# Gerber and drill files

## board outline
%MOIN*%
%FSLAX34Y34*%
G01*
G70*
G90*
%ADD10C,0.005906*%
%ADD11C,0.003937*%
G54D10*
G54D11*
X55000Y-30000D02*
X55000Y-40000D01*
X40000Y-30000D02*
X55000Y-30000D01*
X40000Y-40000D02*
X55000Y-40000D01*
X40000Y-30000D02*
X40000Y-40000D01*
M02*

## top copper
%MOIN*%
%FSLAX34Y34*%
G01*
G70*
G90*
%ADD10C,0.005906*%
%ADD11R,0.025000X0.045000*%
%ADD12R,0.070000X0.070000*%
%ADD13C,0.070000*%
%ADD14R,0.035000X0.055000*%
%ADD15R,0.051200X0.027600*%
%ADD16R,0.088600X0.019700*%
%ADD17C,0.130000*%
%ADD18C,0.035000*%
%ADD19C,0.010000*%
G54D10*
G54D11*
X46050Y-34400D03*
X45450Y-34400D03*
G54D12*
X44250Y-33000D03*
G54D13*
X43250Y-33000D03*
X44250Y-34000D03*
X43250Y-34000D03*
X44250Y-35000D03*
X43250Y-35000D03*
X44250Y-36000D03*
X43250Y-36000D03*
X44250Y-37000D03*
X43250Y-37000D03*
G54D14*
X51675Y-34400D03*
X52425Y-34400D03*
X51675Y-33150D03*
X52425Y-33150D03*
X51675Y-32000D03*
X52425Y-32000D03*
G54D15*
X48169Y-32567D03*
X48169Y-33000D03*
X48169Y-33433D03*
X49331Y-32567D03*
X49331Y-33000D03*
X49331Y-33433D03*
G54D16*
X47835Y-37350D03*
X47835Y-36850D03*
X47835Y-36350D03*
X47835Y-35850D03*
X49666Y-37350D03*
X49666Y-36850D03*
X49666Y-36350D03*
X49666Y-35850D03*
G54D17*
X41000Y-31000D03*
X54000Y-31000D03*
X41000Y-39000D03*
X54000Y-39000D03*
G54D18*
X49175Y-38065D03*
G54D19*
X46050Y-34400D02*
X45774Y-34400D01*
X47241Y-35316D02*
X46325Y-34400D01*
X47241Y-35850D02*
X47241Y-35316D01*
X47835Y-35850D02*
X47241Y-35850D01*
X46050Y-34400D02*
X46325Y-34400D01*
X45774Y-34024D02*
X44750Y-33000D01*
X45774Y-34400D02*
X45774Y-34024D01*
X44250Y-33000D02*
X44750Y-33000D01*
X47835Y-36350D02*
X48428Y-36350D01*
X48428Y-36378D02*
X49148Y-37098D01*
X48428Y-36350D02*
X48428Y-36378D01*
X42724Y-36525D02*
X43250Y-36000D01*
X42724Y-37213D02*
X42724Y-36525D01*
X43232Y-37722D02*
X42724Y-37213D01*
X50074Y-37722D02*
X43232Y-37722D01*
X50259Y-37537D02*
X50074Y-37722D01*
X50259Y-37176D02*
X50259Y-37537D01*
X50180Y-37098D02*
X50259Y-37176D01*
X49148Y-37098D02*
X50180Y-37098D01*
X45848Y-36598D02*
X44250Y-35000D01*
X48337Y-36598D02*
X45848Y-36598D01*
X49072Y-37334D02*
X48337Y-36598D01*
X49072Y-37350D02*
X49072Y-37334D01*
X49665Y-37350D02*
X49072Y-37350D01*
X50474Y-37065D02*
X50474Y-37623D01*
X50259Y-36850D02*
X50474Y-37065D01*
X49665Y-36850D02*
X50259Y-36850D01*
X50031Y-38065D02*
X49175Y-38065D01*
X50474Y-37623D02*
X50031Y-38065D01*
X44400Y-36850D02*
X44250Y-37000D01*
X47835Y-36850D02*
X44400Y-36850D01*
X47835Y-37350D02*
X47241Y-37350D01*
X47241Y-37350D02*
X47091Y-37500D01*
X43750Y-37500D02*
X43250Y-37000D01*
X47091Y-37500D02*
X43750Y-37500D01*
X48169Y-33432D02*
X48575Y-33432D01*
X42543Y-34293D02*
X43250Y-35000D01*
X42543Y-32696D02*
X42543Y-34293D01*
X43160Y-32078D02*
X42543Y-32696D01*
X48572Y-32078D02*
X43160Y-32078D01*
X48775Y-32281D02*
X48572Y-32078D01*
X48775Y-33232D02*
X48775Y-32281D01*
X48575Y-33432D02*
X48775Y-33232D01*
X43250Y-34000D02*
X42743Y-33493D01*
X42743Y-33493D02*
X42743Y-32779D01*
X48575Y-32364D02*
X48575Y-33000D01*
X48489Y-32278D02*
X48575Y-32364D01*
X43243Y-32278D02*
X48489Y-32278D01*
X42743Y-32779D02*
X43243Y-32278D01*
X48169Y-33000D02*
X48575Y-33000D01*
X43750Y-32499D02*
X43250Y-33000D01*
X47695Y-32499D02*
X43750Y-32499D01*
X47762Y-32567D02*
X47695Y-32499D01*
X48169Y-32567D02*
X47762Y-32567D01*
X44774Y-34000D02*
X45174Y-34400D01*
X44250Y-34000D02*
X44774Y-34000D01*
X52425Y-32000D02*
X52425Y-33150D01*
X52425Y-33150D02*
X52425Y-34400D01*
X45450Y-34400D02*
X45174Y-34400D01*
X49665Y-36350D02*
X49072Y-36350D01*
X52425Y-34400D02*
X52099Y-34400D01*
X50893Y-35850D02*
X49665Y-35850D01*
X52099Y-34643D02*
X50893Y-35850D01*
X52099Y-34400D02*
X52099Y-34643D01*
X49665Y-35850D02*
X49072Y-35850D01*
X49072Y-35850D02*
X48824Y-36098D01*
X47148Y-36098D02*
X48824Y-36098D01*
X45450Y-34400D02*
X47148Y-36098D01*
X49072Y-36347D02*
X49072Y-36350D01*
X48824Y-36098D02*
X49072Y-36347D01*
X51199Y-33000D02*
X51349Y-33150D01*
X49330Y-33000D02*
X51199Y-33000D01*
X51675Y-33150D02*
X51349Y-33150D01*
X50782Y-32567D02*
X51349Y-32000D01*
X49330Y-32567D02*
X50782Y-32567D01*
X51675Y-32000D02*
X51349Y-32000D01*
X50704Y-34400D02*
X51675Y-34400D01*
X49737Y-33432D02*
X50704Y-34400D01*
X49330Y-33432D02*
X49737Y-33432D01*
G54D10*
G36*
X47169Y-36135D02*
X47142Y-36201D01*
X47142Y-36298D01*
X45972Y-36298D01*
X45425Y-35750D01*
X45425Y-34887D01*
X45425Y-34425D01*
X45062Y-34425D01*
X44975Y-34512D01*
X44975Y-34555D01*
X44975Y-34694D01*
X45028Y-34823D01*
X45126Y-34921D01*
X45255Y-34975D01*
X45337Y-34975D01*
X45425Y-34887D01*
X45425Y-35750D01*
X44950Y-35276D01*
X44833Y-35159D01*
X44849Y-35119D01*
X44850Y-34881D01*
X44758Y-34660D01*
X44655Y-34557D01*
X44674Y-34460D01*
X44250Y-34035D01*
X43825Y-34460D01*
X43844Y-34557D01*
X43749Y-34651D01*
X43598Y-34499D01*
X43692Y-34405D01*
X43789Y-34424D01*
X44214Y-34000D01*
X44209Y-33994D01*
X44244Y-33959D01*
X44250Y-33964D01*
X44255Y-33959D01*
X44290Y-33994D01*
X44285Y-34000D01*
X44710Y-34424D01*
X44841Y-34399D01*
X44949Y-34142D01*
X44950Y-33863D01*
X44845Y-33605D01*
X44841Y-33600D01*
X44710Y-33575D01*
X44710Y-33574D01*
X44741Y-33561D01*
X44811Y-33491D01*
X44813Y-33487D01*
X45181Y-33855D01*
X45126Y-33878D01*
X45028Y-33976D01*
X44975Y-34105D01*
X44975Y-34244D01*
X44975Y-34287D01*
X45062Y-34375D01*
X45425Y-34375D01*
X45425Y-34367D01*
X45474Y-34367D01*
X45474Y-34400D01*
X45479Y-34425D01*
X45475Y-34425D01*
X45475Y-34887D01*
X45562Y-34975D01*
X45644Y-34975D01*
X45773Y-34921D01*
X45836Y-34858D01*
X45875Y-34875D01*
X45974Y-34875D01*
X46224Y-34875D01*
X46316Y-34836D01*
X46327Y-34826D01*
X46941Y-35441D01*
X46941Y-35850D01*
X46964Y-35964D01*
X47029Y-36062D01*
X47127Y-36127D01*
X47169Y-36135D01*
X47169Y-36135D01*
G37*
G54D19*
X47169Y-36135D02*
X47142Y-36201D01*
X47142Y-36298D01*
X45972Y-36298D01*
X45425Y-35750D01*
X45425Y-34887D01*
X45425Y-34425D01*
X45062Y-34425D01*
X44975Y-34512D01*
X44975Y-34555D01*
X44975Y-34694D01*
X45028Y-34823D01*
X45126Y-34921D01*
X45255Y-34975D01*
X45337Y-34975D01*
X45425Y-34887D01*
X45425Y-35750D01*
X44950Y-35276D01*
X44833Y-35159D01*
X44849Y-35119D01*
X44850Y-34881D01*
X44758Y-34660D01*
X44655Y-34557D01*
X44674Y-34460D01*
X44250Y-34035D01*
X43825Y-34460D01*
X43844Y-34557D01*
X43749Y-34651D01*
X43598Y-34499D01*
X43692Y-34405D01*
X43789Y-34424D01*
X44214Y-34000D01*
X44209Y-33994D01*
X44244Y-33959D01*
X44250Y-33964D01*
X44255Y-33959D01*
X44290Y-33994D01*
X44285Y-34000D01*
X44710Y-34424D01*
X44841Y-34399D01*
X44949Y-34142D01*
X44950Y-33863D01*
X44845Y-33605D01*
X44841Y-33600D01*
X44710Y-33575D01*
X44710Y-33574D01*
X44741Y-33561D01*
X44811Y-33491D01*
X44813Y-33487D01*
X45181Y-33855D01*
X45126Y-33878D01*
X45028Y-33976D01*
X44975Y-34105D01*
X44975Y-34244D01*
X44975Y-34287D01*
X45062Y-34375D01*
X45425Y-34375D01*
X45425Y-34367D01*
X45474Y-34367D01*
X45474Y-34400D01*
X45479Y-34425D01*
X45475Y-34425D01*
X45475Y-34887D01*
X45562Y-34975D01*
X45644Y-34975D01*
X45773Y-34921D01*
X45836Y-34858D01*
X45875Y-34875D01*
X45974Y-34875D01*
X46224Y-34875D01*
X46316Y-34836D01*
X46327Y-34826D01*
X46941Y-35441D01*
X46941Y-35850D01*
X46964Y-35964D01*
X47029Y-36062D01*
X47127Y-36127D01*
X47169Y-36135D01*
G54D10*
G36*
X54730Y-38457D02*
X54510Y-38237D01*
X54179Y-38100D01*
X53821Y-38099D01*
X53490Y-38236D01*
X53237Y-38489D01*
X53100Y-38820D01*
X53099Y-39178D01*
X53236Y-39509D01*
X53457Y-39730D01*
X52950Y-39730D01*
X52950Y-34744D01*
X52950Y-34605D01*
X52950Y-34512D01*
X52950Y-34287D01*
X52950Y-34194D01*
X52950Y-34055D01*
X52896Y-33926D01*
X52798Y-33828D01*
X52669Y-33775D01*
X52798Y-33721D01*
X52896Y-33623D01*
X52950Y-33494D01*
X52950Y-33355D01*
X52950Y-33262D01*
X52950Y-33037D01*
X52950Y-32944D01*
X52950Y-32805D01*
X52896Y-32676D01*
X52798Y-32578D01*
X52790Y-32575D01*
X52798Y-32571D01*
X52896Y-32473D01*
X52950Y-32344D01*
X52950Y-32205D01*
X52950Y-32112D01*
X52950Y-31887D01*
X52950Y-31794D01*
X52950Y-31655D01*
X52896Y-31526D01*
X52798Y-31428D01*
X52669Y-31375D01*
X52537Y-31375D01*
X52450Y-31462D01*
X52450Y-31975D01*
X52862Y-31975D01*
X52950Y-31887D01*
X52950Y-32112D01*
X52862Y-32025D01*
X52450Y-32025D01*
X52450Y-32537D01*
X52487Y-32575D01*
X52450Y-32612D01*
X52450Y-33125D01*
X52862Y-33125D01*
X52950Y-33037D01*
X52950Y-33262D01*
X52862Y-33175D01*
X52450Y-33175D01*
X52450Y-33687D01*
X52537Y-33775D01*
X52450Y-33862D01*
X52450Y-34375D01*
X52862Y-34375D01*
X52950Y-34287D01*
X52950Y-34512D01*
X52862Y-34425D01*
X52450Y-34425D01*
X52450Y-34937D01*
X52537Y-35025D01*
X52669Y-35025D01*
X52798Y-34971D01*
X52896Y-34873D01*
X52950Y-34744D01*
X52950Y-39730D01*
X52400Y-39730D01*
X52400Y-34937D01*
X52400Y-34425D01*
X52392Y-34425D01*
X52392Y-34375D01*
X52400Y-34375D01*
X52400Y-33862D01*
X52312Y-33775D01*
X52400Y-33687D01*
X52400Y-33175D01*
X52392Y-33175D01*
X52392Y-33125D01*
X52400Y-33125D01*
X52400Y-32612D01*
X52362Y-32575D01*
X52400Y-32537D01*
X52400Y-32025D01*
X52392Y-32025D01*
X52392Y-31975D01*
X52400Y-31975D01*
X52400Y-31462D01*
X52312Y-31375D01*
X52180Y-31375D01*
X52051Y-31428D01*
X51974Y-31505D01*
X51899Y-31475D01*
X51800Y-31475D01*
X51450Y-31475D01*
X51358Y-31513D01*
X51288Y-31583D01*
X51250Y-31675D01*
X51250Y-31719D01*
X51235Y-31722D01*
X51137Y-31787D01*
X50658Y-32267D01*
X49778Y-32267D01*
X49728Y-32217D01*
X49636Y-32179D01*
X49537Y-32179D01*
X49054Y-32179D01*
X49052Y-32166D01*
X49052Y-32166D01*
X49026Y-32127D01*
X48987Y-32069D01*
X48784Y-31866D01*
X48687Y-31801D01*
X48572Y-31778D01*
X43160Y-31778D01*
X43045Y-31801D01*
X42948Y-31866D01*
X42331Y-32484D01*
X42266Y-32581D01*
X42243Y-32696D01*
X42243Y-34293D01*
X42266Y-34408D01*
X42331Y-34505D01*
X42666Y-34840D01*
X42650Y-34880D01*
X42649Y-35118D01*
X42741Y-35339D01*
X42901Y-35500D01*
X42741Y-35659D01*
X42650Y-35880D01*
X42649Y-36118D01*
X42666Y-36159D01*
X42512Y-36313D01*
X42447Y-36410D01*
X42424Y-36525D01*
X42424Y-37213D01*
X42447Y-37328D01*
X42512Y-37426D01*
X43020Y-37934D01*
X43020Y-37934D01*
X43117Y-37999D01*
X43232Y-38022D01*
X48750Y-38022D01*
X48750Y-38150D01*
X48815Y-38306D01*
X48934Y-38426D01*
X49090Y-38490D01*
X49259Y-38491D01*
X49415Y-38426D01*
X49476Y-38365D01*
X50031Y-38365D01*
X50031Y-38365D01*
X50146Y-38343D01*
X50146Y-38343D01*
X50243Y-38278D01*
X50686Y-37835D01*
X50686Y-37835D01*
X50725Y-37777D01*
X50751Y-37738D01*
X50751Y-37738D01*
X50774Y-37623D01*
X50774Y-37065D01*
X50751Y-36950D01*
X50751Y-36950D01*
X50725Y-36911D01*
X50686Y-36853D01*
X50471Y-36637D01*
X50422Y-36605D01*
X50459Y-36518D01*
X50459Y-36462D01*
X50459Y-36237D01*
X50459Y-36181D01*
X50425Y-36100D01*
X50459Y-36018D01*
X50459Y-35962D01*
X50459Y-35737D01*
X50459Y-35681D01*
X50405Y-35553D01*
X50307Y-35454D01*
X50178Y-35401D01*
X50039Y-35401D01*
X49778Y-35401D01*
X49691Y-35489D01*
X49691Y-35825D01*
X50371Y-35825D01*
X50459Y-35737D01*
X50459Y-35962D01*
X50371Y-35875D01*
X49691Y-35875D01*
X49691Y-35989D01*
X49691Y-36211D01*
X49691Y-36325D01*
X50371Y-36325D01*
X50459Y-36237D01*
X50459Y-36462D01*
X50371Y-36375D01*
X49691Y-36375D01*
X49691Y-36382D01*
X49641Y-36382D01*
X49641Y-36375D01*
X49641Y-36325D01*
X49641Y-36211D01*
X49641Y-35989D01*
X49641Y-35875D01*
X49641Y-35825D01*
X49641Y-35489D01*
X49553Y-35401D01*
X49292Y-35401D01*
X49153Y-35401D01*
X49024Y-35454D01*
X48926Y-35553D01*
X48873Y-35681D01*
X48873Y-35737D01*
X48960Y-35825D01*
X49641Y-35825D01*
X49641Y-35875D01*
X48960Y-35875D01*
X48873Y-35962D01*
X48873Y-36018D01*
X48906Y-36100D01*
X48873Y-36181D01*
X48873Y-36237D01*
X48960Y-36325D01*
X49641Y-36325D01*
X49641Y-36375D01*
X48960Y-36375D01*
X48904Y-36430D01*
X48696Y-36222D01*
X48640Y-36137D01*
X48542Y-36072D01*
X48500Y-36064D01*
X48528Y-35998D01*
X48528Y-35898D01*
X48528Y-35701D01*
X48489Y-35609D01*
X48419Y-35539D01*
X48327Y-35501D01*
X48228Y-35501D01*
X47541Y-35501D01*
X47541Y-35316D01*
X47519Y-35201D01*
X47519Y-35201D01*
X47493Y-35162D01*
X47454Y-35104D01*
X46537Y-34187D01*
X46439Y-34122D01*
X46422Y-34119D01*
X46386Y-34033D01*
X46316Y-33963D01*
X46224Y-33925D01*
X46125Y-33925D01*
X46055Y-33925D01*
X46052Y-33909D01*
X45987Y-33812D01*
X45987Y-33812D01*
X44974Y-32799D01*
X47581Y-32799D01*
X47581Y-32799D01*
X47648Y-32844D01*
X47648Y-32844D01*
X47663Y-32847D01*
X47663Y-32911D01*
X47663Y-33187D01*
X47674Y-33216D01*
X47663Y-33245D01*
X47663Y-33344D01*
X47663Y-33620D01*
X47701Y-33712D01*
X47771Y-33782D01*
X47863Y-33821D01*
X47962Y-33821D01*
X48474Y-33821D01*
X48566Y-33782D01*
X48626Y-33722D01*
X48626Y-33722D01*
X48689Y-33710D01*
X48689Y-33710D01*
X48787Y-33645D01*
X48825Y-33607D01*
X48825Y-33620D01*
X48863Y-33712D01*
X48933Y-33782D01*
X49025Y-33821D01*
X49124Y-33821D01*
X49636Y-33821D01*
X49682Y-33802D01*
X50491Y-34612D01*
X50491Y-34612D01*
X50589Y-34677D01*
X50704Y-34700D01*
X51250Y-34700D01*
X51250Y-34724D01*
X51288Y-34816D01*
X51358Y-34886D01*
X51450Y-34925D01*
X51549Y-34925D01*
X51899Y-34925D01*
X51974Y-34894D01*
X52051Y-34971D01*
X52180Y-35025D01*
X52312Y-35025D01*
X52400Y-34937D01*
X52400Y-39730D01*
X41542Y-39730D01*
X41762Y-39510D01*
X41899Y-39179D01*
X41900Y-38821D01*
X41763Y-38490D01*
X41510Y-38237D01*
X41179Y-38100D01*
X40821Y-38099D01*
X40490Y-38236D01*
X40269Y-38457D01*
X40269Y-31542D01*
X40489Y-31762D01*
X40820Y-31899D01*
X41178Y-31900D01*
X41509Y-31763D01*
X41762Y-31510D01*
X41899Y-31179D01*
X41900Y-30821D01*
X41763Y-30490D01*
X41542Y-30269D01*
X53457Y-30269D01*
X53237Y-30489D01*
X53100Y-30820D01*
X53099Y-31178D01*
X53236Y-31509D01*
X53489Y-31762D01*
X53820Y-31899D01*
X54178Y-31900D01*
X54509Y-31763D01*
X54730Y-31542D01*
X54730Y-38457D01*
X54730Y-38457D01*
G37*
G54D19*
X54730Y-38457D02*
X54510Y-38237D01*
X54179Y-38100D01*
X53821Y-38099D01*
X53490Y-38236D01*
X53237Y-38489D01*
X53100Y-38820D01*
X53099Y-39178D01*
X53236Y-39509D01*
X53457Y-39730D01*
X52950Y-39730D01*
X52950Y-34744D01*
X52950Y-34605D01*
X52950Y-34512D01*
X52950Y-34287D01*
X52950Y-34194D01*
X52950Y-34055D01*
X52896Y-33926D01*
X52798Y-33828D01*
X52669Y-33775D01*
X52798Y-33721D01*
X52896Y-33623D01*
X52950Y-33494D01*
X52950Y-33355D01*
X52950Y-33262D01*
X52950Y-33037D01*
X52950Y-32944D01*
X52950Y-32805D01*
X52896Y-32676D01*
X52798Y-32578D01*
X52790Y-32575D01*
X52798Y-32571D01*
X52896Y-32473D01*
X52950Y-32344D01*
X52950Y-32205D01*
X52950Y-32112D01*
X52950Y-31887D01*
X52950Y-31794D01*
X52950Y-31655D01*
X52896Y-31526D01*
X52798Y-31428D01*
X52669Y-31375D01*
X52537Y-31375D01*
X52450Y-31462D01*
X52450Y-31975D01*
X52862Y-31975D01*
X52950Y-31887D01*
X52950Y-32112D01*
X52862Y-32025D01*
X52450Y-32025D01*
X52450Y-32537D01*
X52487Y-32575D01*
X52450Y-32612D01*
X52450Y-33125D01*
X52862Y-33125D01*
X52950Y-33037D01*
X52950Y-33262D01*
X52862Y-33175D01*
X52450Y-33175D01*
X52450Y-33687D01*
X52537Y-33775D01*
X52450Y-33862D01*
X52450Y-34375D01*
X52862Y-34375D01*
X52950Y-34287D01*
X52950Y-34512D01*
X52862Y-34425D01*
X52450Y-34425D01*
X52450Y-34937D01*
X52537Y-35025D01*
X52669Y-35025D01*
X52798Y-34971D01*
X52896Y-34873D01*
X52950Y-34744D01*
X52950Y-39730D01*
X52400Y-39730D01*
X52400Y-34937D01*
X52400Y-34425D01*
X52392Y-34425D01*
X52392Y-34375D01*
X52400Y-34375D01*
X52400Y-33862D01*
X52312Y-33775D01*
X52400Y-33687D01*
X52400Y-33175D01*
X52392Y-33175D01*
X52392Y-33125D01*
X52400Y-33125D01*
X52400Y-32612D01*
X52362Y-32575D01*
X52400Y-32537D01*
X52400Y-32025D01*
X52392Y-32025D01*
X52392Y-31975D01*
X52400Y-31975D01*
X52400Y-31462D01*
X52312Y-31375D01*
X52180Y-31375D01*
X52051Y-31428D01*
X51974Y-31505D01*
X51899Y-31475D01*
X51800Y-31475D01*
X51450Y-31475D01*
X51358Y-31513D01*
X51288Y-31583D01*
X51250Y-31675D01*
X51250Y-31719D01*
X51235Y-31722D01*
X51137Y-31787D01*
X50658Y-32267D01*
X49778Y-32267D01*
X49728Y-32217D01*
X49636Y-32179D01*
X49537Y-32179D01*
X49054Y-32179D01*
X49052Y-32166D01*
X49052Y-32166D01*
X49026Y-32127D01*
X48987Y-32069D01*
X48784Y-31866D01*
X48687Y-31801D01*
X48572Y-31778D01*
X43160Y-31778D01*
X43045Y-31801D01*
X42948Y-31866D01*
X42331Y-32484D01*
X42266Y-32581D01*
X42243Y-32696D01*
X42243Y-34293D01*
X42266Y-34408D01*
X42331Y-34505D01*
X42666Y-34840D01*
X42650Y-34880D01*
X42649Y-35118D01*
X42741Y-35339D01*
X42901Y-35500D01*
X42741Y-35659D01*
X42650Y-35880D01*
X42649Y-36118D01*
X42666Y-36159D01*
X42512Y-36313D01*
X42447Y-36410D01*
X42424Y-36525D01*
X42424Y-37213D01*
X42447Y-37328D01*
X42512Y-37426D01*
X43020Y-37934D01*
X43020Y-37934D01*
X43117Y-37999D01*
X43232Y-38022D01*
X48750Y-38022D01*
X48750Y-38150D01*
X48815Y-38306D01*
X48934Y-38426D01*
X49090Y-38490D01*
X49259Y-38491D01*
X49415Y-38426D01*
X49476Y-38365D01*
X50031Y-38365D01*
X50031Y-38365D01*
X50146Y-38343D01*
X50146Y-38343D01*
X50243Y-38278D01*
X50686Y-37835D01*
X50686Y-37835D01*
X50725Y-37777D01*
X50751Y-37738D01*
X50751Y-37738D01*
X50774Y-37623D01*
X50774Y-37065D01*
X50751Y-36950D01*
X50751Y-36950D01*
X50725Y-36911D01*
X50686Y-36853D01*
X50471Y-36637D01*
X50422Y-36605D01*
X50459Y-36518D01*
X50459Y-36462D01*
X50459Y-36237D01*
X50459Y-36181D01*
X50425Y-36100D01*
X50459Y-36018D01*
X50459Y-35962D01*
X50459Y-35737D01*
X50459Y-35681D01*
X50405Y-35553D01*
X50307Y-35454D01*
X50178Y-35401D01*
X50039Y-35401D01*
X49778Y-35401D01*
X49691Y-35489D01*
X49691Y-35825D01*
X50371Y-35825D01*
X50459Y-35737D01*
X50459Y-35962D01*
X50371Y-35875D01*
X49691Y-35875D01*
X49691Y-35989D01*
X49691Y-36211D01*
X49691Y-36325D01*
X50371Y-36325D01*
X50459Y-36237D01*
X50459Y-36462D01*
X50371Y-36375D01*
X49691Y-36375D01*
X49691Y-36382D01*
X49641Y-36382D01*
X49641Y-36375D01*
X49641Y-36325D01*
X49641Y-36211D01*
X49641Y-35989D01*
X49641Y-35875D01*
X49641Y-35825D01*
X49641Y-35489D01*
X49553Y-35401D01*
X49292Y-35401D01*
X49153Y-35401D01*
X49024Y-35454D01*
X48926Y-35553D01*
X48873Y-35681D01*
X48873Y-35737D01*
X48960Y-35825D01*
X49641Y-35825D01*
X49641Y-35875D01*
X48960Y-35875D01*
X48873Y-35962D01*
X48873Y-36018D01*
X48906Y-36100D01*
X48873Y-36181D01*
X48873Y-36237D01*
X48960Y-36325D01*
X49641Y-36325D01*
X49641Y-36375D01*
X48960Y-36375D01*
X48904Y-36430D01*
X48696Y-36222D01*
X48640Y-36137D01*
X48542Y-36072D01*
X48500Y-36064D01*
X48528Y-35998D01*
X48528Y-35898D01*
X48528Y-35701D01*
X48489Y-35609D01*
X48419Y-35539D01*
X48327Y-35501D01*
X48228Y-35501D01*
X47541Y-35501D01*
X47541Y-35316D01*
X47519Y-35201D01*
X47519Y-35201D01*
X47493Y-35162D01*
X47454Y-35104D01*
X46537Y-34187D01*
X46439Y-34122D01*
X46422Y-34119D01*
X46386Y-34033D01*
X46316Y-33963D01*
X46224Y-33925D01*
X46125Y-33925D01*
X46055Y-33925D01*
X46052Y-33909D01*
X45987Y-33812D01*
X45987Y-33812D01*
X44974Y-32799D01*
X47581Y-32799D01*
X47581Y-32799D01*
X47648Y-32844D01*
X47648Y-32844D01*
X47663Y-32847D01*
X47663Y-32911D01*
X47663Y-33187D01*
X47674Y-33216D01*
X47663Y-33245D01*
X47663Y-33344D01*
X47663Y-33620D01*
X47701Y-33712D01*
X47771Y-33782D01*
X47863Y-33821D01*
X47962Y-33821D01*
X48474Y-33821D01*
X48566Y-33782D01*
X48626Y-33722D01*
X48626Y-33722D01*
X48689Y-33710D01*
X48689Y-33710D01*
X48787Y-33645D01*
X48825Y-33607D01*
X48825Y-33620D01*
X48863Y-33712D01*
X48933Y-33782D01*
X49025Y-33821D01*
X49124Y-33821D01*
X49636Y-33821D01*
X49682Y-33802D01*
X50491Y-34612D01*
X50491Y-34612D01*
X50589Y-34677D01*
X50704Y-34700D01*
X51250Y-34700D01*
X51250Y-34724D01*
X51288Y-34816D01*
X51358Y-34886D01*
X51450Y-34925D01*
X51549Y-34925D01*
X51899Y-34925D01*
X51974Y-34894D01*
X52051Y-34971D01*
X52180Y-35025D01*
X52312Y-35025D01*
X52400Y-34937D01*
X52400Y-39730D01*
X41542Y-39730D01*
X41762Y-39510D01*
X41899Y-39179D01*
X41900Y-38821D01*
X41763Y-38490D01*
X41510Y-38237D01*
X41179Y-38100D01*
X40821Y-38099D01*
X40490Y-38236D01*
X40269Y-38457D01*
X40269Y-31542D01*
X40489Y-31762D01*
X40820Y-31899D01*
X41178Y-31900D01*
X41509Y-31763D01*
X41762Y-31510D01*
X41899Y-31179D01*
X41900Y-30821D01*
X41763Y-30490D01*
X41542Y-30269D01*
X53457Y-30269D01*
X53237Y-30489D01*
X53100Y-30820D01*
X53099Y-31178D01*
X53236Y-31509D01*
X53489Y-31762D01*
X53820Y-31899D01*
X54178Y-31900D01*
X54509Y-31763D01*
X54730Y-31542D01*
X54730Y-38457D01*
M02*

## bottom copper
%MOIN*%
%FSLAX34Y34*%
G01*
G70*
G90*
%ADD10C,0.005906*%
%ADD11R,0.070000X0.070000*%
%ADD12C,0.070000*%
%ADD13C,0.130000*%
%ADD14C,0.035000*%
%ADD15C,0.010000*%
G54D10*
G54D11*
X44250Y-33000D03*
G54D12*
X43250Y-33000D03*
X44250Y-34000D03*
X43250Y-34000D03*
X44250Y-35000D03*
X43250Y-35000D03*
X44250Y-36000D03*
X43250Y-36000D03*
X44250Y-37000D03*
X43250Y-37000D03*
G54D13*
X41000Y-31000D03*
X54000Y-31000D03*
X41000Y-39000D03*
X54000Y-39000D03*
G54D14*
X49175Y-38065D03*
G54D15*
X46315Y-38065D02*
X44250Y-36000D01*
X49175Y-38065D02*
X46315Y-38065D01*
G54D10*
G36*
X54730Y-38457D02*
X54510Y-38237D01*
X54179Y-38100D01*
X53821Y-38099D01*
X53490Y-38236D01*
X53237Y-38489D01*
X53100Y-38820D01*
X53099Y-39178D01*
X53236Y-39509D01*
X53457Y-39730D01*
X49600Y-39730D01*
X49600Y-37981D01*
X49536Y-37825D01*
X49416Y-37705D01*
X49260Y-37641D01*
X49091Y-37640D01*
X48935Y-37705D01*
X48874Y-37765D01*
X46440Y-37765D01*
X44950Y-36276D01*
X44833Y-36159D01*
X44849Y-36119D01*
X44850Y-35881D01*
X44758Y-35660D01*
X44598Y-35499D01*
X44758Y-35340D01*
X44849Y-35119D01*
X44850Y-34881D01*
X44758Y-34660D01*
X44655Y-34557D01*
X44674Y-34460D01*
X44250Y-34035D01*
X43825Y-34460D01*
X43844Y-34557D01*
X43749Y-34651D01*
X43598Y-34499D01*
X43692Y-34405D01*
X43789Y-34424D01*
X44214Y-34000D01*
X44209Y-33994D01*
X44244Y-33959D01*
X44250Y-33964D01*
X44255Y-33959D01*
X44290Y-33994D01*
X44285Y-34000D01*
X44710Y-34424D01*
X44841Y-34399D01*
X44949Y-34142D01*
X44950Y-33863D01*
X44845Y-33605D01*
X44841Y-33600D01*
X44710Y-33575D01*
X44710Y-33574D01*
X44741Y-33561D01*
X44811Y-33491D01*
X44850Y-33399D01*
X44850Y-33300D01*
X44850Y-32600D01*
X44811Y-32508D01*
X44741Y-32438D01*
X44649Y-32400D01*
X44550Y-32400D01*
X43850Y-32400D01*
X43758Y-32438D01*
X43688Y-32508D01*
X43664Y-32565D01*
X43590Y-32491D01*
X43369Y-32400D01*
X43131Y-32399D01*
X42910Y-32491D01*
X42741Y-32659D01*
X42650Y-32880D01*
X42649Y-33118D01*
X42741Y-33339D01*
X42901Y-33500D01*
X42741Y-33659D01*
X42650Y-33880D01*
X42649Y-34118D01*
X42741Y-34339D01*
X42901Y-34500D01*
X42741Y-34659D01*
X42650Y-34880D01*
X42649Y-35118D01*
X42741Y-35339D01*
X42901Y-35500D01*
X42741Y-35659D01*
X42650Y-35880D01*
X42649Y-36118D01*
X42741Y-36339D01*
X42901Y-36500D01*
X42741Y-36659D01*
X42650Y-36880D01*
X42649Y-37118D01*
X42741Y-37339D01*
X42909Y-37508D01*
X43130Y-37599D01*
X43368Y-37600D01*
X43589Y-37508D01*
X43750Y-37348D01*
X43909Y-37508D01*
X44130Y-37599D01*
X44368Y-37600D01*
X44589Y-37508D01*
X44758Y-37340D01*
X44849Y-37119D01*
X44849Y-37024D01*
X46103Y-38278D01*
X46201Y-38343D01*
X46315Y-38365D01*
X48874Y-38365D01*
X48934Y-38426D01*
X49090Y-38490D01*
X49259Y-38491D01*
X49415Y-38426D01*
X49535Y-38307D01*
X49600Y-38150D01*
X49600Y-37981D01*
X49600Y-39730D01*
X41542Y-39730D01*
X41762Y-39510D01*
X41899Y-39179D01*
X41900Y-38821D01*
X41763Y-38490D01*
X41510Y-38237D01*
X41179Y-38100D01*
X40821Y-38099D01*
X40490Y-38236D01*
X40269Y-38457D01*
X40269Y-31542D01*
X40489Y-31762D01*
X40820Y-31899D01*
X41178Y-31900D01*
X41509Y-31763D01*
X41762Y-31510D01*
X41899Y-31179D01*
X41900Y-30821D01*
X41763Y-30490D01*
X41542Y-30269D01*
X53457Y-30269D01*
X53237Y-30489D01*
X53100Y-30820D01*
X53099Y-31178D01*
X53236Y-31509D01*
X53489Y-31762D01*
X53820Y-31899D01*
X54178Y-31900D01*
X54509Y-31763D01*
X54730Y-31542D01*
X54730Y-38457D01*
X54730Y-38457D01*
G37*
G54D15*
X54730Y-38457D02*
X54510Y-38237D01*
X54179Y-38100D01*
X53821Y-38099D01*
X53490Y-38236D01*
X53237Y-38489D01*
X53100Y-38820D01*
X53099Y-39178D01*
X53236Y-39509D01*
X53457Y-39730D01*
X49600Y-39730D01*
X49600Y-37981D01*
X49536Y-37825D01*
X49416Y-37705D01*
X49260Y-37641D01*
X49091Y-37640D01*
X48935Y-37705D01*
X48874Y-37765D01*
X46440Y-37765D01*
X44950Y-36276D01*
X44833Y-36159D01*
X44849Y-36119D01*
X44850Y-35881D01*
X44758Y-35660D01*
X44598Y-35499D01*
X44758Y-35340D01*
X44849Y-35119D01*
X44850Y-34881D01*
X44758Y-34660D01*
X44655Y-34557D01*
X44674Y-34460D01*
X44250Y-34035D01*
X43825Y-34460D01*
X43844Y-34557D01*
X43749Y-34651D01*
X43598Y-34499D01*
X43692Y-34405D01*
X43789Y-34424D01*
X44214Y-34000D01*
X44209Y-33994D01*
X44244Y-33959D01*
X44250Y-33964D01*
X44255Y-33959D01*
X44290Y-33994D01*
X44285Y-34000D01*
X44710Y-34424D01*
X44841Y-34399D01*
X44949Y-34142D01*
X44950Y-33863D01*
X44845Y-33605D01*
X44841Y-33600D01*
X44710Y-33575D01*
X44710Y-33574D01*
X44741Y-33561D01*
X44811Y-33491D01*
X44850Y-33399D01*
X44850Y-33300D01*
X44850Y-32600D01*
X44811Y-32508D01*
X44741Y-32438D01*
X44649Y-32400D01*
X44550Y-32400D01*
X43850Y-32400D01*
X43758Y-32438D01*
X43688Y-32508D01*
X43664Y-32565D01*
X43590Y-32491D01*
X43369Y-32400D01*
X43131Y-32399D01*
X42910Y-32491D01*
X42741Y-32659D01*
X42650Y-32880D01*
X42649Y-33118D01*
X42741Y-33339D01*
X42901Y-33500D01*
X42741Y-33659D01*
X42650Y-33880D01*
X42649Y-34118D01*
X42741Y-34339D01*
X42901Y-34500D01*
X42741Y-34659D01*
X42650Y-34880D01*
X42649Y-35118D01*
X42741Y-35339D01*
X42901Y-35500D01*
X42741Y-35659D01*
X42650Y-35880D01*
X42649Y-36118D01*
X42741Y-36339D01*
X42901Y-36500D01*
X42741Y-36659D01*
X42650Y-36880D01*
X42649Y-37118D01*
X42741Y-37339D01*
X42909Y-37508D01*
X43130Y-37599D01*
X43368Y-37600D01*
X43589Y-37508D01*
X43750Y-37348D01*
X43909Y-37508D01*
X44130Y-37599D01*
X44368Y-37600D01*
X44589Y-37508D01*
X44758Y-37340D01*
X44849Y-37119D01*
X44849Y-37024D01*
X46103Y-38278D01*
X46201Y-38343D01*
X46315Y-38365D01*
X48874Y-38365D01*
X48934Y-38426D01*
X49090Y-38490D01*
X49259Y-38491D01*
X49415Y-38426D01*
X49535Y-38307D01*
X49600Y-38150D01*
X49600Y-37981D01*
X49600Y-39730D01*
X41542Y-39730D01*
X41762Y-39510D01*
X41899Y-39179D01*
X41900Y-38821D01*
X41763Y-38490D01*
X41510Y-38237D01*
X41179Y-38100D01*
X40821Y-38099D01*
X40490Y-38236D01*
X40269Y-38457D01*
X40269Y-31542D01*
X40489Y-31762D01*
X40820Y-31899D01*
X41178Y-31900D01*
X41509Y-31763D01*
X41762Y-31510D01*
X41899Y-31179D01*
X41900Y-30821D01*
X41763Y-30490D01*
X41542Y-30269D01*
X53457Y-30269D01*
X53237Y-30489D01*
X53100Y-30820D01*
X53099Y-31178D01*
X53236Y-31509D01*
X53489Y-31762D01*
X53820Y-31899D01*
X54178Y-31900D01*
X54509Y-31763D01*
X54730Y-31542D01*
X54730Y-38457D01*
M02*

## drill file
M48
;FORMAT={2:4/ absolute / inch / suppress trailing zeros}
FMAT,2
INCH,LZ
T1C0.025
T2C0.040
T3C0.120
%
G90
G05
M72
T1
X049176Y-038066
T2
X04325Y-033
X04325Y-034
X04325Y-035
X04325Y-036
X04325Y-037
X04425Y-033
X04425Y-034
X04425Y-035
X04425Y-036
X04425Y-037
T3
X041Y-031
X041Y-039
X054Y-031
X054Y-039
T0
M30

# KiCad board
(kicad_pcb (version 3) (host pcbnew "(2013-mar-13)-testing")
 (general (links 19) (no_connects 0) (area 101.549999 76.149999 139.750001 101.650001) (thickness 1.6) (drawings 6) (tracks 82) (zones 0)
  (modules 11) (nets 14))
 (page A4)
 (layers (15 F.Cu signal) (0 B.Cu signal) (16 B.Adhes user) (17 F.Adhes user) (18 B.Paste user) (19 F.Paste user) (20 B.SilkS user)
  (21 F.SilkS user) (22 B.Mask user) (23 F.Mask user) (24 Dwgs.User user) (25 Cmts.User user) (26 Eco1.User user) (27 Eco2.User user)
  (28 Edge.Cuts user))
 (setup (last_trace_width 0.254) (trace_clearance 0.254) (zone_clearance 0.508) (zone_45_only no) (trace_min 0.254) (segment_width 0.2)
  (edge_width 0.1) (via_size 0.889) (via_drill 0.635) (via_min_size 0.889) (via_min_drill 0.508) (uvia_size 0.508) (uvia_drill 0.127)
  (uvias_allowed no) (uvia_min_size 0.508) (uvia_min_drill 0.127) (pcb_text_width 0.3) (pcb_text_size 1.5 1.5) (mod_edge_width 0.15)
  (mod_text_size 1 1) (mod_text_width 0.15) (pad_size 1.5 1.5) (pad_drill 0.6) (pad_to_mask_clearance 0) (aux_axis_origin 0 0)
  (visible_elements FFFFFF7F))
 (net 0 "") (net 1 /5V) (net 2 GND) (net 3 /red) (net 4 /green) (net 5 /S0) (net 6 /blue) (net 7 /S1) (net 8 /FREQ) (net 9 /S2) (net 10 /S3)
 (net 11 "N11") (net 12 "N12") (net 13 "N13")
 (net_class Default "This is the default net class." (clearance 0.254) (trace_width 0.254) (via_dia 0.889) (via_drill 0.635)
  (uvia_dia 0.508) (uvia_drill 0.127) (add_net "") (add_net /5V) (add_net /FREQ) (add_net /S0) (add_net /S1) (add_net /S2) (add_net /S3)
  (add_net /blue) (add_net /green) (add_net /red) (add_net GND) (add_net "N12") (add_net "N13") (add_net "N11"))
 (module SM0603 (layer F.Cu) (at 116.205 87.376 180)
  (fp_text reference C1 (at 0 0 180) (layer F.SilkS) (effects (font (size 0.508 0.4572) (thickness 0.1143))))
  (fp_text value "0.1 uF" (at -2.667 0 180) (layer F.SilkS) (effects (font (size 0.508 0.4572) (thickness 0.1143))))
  (pad 1 smd rect (at -0.762 0 180) (size 0.635 1.143) (layers F.Cu F.Paste F.Mask) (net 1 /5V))
  (pad 2 smd rect (at 0.762 0 180) (size 0.635 1.143) (layers F.Cu F.Paste F.Mask) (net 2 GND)))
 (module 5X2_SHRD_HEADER (layer B.Cu) (at 111.125 88.9 270)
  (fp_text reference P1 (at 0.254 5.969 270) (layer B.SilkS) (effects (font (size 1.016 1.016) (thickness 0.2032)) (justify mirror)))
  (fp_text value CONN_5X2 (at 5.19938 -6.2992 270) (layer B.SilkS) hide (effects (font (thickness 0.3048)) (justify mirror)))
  (pad 1 thru_hole rect (at -5.08 -1.27 270) (size 1.778 1.778) (drill 1.016) (layers *.Cu *.Mask B.SilkS) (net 1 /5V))
  (pad 2 thru_hole circle (at -5.08 1.27 270) (size 1.778 1.778) (drill 1.016) (layers *.Cu *.Mask B.SilkS) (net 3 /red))
  (pad 3 thru_hole circle (at -2.54 -1.27 270) (size 1.778 1.778) (drill 1.016) (layers *.Cu *.Mask B.SilkS) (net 2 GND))
  (pad 4 thru_hole circle (at -2.54 1.27 270) (size 1.778 1.778) (drill 1.016) (layers *.Cu *.Mask B.SilkS) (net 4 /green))
  (pad 5 thru_hole circle (at 0 -1.27 270) (size 1.778 1.778) (drill 1.016) (layers *.Cu *.Mask B.SilkS) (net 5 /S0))
  (pad 6 thru_hole circle (at 0 1.27 270) (size 1.778 1.778) (drill 1.016) (layers *.Cu *.Mask B.SilkS) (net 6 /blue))
  (pad 7 thru_hole circle (at 2.54 -1.27 270) (size 1.778 1.778) (drill 1.016) (layers *.Cu *.Mask B.SilkS) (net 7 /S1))
  (pad 8 thru_hole circle (at 2.54 1.27 270) (size 1.778 1.778) (drill 1.016) (layers *.Cu *.Mask B.SilkS) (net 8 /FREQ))
  (pad 9 thru_hole circle (at 5.08 -1.27 270) (size 1.778 1.778) (drill 1.016) (layers *.Cu *.Mask B.SilkS) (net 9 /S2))
  (pad 10 thru_hole circle (at 5.08 1.27 270) (size 1.778 1.778) (drill 1.016) (layers *.Cu *.Mask B.SilkS) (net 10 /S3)))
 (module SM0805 (layer F.Cu) (at 132.207 87.376)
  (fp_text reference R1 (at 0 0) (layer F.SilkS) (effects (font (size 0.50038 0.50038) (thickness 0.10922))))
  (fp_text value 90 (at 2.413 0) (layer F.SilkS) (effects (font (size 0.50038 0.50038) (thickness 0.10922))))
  (pad 1 smd rect (at -0.9525 0) (size 0.889 1.397) (layers F.Cu F.Paste F.Mask) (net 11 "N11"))
  (pad 2 smd rect (at 0.9525 0) (size 0.889 1.397) (layers F.Cu F.Paste F.Mask) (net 2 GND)))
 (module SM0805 (layer F.Cu) (at 132.207 84.201)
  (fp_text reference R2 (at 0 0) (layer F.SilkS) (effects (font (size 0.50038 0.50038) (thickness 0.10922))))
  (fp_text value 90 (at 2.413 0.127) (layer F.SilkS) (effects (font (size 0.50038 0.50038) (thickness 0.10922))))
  (pad 1 smd rect (at -0.9525 0) (size 0.889 1.397) (layers F.Cu F.Paste F.Mask) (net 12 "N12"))
  (pad 2 smd rect (at 0.9525 0) (size 0.889 1.397) (layers F.Cu F.Paste F.Mask) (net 2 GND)))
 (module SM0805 (layer F.Cu) (at 132.207 81.28)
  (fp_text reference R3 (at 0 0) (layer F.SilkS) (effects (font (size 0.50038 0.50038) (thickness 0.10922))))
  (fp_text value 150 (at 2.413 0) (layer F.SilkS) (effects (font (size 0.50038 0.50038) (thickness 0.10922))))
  (pad 1 smd rect (at -0.9525 0) (size 0.889 1.397) (layers F.Cu F.Paste F.Mask) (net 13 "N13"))
  (pad 2 smd rect (at 0.9525 0) (size 0.889 1.397) (layers F.Cu F.Paste F.Mask) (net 2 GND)))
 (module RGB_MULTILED (layer F.Cu) (at 123.825 83.82 180)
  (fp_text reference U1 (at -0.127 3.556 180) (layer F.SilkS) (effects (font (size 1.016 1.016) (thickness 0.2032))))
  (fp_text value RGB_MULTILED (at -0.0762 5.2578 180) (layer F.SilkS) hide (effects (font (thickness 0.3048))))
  (pad A3 smd rect (at 1.47574 1.09982) (size 1.30048 0.70104) (layers F.Cu F.Paste F.Mask) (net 3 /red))
  (pad A2 smd rect (at 1.47574 0) (size 1.30048 0.70104) (layers F.Cu F.Paste F.Mask) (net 4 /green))
  (pad A1 smd rect (at 1.47574 -1.09982) (size 1.30048 0.70104) (layers F.Cu F.Paste F.Mask) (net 6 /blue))
  (pad C3 smd rect (at -1.47574 1.09982) (size 1.30048 0.70104) (layers F.Cu F.Paste F.Mask) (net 13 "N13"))
  (pad C2 smd rect (at -1.47574 0) (size 1.30048 0.70104) (layers F.Cu F.Paste F.Mask) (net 12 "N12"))
  (pad C1 smd rect (at -1.47574 -1.09982) (size 1.30048 0.70104) (layers F.Cu F.Paste F.Mask) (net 11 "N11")))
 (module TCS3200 (layer F.Cu) (at 123.825 92.964 90)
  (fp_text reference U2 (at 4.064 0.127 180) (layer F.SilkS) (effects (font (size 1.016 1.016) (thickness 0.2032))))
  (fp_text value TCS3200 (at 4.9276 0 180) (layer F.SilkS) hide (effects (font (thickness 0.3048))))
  (pad 8 smd rect (at -1.905 -2.3241 90) (size 0.50038 2.25044) (layers F.Cu F.Paste F.Mask) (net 10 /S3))
  (pad 7 smd rect (at -0.635 -2.3241 90) (size 0.50038 2.25044) (layers F.Cu F.Paste F.Mask) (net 9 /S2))
  (pad 6 smd rect (at 0.635 -2.3241 90) (size 0.50038 2.25044) (layers F.Cu F.Paste F.Mask) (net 8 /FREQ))
  (pad 5 smd rect (at 1.905 -2.3241 90) (size 0.50038 2.25044) (layers F.Cu F.Paste F.Mask) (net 1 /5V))
  (pad 1 smd rect (at -1.905 2.32664 90) (size 0.50038 2.25044) (layers F.Cu F.Paste F.Mask) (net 5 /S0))
  (pad 2 smd rect (at -0.635 2.32664 90) (size 0.50038 2.25044) (layers F.Cu F.Paste F.Mask) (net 7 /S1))
  (pad 3 smd rect (at 0.635 2.32664 90) (size 0.50038 2.25044) (layers F.Cu F.Paste F.Mask) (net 2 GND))
  (pad 4 smd rect (at 1.905 2.32664 90) (size 0.50038 2.25044) (layers F.Cu F.Paste F.Mask) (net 2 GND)))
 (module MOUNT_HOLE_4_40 (layer F.Cu) (at 104.14 78.74)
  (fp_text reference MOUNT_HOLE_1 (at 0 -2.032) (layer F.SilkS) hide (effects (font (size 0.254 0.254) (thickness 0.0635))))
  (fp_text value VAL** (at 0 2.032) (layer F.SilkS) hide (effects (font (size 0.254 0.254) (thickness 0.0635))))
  (pad "" thru_hole circle (at 0 0) (size 3.302 3.302) (drill 3.048) (layers *.Cu *.SilkS *.Mask)))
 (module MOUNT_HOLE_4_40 (layer F.Cu) (at 137.16 78.74)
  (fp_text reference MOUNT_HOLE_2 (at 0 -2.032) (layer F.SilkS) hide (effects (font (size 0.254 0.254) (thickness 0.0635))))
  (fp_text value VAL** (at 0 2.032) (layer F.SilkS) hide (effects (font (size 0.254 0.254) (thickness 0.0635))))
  (pad "" thru_hole circle (at 0 0) (size 3.302 3.302) (drill 3.048) (layers *.Cu *.SilkS *.Mask)))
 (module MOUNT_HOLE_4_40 (layer F.Cu) (at 104.14 99.06)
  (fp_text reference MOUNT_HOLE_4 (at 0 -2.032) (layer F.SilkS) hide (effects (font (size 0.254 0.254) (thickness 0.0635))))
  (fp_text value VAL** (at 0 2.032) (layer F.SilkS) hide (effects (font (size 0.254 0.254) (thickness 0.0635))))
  (pad "" thru_hole circle (at 0 0) (size 3.302 3.302) (drill 3.048) (layers *.Cu *.SilkS *.Mask)))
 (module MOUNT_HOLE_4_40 (layer F.Cu) (at 137.16 99.06)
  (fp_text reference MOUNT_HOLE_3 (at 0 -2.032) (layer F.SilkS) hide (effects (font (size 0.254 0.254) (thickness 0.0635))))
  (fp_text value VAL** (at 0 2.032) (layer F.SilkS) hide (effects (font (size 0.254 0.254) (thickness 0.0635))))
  (pad "" thru_hole circle (at 0 0) (size 3.302 3.302) (drill 3.048) (layers *.Cu *.SilkS *.Mask)))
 (gr_line (start 139.7 76.2) (end 139.7 101.6) (angle 90) (layer Edge.Cuts) (width 0.1))
 (gr_line (start 101.6 76.2) (end 139.7 76.2) (angle 90) (layer Edge.Cuts) (width 0.1))
 (gr_line (start 101.6 101.6) (end 139.7 101.6) (angle 90) (layer Edge.Cuts) (width 0.1))
 (gr_line (start 101.6 76.2) (end 101.6 101.6) (angle 90) (layer Edge.Cuts) (width 0.1))
 (segment (start 116.967 87.376) (end 116.2682 87.376) (width 0.254) (layer F.Cu) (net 1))
 (segment (start 119.9944 89.7046) (end 117.6658 87.376) (width 0.254) (layer F.Cu) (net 1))
 (segment (start 119.9944 91.059) (end 119.9944 89.7046) (width 0.254) (layer F.Cu) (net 1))
 (segment (start 121.5009 91.059) (end 119.9944 91.059) (width 0.254) (layer F.Cu) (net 1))
 (segment (start 116.967 87.376) (end 117.6658 87.376) (width 0.254) (layer F.Cu) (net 1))
 (segment (start 116.2682 86.4229) (end 113.6653 83.82) (width 0.254) (layer F.Cu) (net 1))
 (segment (start 116.2682 87.376) (end 116.2682 86.4229) (width 0.254) (layer F.Cu) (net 1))
 (segment (start 112.395 83.82) (end 113.6653 83.82) (width 0.254) (layer F.Cu) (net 1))
 (segment (start 121.5009 92.329) (end 123.0074 92.329) (width 0.254) (layer F.Cu) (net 8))
 (segment (start 123.0074 92.4005) (end 124.8375 94.2306) (width 0.254) (layer F.Cu) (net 8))
 (segment (start 123.0074 92.329) (end 123.0074 92.4005) (width 0.254) (layer F.Cu) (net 8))
 (segment (start 108.5196 92.7754) (end 109.855 91.44) (width 0.254) (layer F.Cu) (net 8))
 (segment (start 108.5196 94.5235) (end 108.5196 92.7754) (width 0.254) (layer F.Cu) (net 8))
 (segment (start 109.811 95.8149) (end 108.5196 94.5235) (width 0.254) (layer F.Cu) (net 8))
 (segment (start 127.188 95.8149) (end 109.811 95.8149) (width 0.254) (layer F.Cu) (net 8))
 (segment (start 127.6582 95.3447) (end 127.188 95.8149) (width 0.254) (layer F.Cu) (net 8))
 (segment (start 127.6582 94.4293) (end 127.6582 95.3447) (width 0.254) (layer F.Cu) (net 8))
 (segment (start 127.4595 94.2306) (end 127.6582 94.4293) (width 0.254) (layer F.Cu) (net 8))
 (segment (start 124.8375 94.2306) (end 127.4595 94.2306) (width 0.254) (layer F.Cu) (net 8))
 (segment (start 116.4555 92.9605) (end 112.395 88.9) (width 0.254) (layer F.Cu) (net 5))
 (segment (start 122.777 92.9605) (end 116.4555 92.9605) (width 0.254) (layer F.Cu) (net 5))
 (segment (start 124.6451 94.8286) (end 122.777 92.9605) (width 0.254) (layer F.Cu) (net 5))
 (segment (start 124.6451 94.869) (end 124.6451 94.8286) (width 0.254) (layer F.Cu) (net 5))
 (segment (start 126.1516 94.869) (end 124.6451 94.869) (width 0.254) (layer F.Cu) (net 5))
 (segment (start 128.2046 94.1455) (end 128.2046 95.5639) (width 0.254) (layer F.Cu) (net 7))
 (segment (start 127.6581 93.599) (end 128.2046 94.1455) (width 0.254) (layer F.Cu) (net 7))
 (segment (start 126.1516 93.599) (end 127.6581 93.599) (width 0.254) (layer F.Cu) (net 7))
 (segment (start 127.0809 96.6876) (end 124.9058 96.6876) (width 0.254) (layer F.Cu) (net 7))
 (segment (start 128.2046 95.5639) (end 127.0809 96.6876) (width 0.254) (layer F.Cu) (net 7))
 (via (at 124.9058 96.6876) (size 0.889) (layers F.Cu B.Cu) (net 7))
 (segment (start 117.6426 96.6876) (end 112.395 91.44) (width 0.254) (layer B.Cu) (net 7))
 (segment (start 124.9058 96.6876) (end 117.6426 96.6876) (width 0.254) (layer B.Cu) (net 7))
 (segment (start 112.776 93.599) (end 112.395 93.98) (width 0.254) (layer F.Cu) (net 9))
 (segment (start 121.5009 93.599) (end 112.776 93.599) (width 0.254) (layer F.Cu) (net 9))
 (segment (start 121.5009 94.869) (end 119.9944 94.869) (width 0.254) (layer F.Cu) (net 10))
 (segment (start 119.9944 94.869) (end 119.6116 95.2518) (width 0.254) (layer F.Cu) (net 10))
 (segment (start 111.1268 95.2518) (end 109.855 93.98) (width 0.254) (layer F.Cu) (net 10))
 (segment (start 119.6116 95.2518) (end 111.1268 95.2518) (width 0.254) (layer F.Cu) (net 10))
 (segment (start 122.3493 84.9198) (end 123.3808 84.9198) (width 0.254) (layer F.Cu) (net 6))
 (segment (start 108.0599 87.1049) (end 109.855 88.9) (width 0.254) (layer F.Cu) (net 6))
 (segment (start 108.0599 83.0483) (end 108.0599 87.1049) (width 0.254) (layer F.Cu) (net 6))
 (segment (start 109.6282 81.48) (end 108.0599 83.0483) (width 0.254) (layer F.Cu) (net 6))
 (segment (start 123.3749 81.48) (end 109.6282 81.48) (width 0.254) (layer F.Cu) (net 6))
 (segment (start 123.8891 81.9942) (end 123.3749 81.48) (width 0.254) (layer F.Cu) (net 6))
 (segment (start 123.8891 84.4115) (end 123.8891 81.9942) (width 0.254) (layer F.Cu) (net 6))
 (segment (start 123.3808 84.9198) (end 123.8891 84.4115) (width 0.254) (layer F.Cu) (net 6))
 (segment (start 109.855 86.36) (end 108.5682 85.0732) (width 0.254) (layer F.Cu) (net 4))
 (segment (start 108.5682 85.0732) (end 108.5682 83.2588) (width 0.254) (layer F.Cu) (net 4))
 (segment (start 123.3808 82.2047) (end 123.3808 83.82) (width 0.254) (layer F.Cu) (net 4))
 (segment (start 123.1644 81.9883) (end 123.3808 82.2047) (width 0.254) (layer F.Cu) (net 4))
 (segment (start 109.8387 81.9883) (end 123.1644 81.9883) (width 0.254) (layer F.Cu) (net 4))
 (segment (start 108.5682 83.2588) (end 109.8387 81.9883) (width 0.254) (layer F.Cu) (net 4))
 (segment (start 122.3493 83.82) (end 123.3808 83.82) (width 0.254) (layer F.Cu) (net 4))
 (segment (start 111.1254 82.5496) (end 109.855 83.82) (width 0.254) (layer F.Cu) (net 3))
 (segment (start 121.1472 82.5496) (end 111.1254 82.5496) (width 0.254) (layer F.Cu) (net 3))
 (segment (start 121.3178 82.7202) (end 121.1472 82.5496) (width 0.254) (layer F.Cu) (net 3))
 (segment (start 122.3493 82.7202) (end 121.3178 82.7202) (width 0.254) (layer F.Cu) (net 3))
 (segment (start 113.7282 86.36) (end 114.7442 87.376) (width 0.254) (layer F.Cu) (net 2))
 (segment (start 112.395 86.36) (end 113.7282 86.36) (width 0.254) (layer F.Cu) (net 2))
 (segment (start 133.1595 81.28) (end 133.1595 84.201) (width 0.254) (layer F.Cu) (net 2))
 (segment (start 133.1595 84.201) (end 133.1595 87.376) (width 0.254) (layer F.Cu) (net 2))
 (segment (start 115.443 87.376) (end 114.7442 87.376) (width 0.254) (layer F.Cu) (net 2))
 (segment (start 126.1516 92.329) (end 124.6451 92.329) (width 0.254) (layer F.Cu) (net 2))
 (segment (start 133.1595 87.376) (end 132.3337 87.376) (width 0.254) (layer F.Cu) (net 2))
 (segment (start 129.27 91.059) (end 126.1516 91.059) (width 0.254) (layer F.Cu) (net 2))
 (segment (start 132.3337 87.9953) (end 129.27 91.059) (width 0.254) (layer F.Cu) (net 2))
 (segment (start 132.3337 87.376) (end 132.3337 87.9953) (width 0.254) (layer F.Cu) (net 2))
 (segment (start 126.1516 91.059) (end 124.6451 91.059) (width 0.254) (layer F.Cu) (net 2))
 (segment (start 124.6451 91.059) (end 124.0136 91.6905) (width 0.254) (layer F.Cu) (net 2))
 (segment (start 119.7575 91.6905) (end 124.0136 91.6905) (width 0.254) (layer F.Cu) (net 2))
 (segment (start 115.443 87.376) (end 119.7575 91.6905) (width 0.254) (layer F.Cu) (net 2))
 (segment (start 124.6451 92.322) (end 124.6451 92.329) (width 0.254) (layer F.Cu) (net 2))
 (segment (start 124.0136 91.6905) (end 124.6451 92.322) (width 0.254) (layer F.Cu) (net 2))
 (segment (start 130.0477 83.82) (end 130.4287 84.201) (width 0.254) (layer F.Cu) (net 12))
 (segment (start 125.3007 83.82) (end 130.0477 83.82) (width 0.254) (layer F.Cu) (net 12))
 (segment (start 131.2545 84.201) (end 130.4287 84.201) (width 0.254) (layer F.Cu) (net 12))
 (segment (start 128.9885 82.7202) (end 130.4287 81.28) (width 0.254) (layer F.Cu) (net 13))
 (segment (start 125.3007 82.7202) (end 128.9885 82.7202) (width 0.254) (layer F.Cu) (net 13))
 (segment (start 131.2545 81.28) (end 130.4287 81.28) (width 0.254) (layer F.Cu) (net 13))
 (segment (start 128.7884 87.376) (end 131.2545 87.376) (width 0.254) (layer F.Cu) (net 11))
 (segment (start 126.3322 84.9198) (end 128.7884 87.376) (width 0.254) (layer F.Cu) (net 11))
 (segment (start 125.3007 84.9198) (end 126.3322 84.9198) (width 0.254) (layer F.Cu) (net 11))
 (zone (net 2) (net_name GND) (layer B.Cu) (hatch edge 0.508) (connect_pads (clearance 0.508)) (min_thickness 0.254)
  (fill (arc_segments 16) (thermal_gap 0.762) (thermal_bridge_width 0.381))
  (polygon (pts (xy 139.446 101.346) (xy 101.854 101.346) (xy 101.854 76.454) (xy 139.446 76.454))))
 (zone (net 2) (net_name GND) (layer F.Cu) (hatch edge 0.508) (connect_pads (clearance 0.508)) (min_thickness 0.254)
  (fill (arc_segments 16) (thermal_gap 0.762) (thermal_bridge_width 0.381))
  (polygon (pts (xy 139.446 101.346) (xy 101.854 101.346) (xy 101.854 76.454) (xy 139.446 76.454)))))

